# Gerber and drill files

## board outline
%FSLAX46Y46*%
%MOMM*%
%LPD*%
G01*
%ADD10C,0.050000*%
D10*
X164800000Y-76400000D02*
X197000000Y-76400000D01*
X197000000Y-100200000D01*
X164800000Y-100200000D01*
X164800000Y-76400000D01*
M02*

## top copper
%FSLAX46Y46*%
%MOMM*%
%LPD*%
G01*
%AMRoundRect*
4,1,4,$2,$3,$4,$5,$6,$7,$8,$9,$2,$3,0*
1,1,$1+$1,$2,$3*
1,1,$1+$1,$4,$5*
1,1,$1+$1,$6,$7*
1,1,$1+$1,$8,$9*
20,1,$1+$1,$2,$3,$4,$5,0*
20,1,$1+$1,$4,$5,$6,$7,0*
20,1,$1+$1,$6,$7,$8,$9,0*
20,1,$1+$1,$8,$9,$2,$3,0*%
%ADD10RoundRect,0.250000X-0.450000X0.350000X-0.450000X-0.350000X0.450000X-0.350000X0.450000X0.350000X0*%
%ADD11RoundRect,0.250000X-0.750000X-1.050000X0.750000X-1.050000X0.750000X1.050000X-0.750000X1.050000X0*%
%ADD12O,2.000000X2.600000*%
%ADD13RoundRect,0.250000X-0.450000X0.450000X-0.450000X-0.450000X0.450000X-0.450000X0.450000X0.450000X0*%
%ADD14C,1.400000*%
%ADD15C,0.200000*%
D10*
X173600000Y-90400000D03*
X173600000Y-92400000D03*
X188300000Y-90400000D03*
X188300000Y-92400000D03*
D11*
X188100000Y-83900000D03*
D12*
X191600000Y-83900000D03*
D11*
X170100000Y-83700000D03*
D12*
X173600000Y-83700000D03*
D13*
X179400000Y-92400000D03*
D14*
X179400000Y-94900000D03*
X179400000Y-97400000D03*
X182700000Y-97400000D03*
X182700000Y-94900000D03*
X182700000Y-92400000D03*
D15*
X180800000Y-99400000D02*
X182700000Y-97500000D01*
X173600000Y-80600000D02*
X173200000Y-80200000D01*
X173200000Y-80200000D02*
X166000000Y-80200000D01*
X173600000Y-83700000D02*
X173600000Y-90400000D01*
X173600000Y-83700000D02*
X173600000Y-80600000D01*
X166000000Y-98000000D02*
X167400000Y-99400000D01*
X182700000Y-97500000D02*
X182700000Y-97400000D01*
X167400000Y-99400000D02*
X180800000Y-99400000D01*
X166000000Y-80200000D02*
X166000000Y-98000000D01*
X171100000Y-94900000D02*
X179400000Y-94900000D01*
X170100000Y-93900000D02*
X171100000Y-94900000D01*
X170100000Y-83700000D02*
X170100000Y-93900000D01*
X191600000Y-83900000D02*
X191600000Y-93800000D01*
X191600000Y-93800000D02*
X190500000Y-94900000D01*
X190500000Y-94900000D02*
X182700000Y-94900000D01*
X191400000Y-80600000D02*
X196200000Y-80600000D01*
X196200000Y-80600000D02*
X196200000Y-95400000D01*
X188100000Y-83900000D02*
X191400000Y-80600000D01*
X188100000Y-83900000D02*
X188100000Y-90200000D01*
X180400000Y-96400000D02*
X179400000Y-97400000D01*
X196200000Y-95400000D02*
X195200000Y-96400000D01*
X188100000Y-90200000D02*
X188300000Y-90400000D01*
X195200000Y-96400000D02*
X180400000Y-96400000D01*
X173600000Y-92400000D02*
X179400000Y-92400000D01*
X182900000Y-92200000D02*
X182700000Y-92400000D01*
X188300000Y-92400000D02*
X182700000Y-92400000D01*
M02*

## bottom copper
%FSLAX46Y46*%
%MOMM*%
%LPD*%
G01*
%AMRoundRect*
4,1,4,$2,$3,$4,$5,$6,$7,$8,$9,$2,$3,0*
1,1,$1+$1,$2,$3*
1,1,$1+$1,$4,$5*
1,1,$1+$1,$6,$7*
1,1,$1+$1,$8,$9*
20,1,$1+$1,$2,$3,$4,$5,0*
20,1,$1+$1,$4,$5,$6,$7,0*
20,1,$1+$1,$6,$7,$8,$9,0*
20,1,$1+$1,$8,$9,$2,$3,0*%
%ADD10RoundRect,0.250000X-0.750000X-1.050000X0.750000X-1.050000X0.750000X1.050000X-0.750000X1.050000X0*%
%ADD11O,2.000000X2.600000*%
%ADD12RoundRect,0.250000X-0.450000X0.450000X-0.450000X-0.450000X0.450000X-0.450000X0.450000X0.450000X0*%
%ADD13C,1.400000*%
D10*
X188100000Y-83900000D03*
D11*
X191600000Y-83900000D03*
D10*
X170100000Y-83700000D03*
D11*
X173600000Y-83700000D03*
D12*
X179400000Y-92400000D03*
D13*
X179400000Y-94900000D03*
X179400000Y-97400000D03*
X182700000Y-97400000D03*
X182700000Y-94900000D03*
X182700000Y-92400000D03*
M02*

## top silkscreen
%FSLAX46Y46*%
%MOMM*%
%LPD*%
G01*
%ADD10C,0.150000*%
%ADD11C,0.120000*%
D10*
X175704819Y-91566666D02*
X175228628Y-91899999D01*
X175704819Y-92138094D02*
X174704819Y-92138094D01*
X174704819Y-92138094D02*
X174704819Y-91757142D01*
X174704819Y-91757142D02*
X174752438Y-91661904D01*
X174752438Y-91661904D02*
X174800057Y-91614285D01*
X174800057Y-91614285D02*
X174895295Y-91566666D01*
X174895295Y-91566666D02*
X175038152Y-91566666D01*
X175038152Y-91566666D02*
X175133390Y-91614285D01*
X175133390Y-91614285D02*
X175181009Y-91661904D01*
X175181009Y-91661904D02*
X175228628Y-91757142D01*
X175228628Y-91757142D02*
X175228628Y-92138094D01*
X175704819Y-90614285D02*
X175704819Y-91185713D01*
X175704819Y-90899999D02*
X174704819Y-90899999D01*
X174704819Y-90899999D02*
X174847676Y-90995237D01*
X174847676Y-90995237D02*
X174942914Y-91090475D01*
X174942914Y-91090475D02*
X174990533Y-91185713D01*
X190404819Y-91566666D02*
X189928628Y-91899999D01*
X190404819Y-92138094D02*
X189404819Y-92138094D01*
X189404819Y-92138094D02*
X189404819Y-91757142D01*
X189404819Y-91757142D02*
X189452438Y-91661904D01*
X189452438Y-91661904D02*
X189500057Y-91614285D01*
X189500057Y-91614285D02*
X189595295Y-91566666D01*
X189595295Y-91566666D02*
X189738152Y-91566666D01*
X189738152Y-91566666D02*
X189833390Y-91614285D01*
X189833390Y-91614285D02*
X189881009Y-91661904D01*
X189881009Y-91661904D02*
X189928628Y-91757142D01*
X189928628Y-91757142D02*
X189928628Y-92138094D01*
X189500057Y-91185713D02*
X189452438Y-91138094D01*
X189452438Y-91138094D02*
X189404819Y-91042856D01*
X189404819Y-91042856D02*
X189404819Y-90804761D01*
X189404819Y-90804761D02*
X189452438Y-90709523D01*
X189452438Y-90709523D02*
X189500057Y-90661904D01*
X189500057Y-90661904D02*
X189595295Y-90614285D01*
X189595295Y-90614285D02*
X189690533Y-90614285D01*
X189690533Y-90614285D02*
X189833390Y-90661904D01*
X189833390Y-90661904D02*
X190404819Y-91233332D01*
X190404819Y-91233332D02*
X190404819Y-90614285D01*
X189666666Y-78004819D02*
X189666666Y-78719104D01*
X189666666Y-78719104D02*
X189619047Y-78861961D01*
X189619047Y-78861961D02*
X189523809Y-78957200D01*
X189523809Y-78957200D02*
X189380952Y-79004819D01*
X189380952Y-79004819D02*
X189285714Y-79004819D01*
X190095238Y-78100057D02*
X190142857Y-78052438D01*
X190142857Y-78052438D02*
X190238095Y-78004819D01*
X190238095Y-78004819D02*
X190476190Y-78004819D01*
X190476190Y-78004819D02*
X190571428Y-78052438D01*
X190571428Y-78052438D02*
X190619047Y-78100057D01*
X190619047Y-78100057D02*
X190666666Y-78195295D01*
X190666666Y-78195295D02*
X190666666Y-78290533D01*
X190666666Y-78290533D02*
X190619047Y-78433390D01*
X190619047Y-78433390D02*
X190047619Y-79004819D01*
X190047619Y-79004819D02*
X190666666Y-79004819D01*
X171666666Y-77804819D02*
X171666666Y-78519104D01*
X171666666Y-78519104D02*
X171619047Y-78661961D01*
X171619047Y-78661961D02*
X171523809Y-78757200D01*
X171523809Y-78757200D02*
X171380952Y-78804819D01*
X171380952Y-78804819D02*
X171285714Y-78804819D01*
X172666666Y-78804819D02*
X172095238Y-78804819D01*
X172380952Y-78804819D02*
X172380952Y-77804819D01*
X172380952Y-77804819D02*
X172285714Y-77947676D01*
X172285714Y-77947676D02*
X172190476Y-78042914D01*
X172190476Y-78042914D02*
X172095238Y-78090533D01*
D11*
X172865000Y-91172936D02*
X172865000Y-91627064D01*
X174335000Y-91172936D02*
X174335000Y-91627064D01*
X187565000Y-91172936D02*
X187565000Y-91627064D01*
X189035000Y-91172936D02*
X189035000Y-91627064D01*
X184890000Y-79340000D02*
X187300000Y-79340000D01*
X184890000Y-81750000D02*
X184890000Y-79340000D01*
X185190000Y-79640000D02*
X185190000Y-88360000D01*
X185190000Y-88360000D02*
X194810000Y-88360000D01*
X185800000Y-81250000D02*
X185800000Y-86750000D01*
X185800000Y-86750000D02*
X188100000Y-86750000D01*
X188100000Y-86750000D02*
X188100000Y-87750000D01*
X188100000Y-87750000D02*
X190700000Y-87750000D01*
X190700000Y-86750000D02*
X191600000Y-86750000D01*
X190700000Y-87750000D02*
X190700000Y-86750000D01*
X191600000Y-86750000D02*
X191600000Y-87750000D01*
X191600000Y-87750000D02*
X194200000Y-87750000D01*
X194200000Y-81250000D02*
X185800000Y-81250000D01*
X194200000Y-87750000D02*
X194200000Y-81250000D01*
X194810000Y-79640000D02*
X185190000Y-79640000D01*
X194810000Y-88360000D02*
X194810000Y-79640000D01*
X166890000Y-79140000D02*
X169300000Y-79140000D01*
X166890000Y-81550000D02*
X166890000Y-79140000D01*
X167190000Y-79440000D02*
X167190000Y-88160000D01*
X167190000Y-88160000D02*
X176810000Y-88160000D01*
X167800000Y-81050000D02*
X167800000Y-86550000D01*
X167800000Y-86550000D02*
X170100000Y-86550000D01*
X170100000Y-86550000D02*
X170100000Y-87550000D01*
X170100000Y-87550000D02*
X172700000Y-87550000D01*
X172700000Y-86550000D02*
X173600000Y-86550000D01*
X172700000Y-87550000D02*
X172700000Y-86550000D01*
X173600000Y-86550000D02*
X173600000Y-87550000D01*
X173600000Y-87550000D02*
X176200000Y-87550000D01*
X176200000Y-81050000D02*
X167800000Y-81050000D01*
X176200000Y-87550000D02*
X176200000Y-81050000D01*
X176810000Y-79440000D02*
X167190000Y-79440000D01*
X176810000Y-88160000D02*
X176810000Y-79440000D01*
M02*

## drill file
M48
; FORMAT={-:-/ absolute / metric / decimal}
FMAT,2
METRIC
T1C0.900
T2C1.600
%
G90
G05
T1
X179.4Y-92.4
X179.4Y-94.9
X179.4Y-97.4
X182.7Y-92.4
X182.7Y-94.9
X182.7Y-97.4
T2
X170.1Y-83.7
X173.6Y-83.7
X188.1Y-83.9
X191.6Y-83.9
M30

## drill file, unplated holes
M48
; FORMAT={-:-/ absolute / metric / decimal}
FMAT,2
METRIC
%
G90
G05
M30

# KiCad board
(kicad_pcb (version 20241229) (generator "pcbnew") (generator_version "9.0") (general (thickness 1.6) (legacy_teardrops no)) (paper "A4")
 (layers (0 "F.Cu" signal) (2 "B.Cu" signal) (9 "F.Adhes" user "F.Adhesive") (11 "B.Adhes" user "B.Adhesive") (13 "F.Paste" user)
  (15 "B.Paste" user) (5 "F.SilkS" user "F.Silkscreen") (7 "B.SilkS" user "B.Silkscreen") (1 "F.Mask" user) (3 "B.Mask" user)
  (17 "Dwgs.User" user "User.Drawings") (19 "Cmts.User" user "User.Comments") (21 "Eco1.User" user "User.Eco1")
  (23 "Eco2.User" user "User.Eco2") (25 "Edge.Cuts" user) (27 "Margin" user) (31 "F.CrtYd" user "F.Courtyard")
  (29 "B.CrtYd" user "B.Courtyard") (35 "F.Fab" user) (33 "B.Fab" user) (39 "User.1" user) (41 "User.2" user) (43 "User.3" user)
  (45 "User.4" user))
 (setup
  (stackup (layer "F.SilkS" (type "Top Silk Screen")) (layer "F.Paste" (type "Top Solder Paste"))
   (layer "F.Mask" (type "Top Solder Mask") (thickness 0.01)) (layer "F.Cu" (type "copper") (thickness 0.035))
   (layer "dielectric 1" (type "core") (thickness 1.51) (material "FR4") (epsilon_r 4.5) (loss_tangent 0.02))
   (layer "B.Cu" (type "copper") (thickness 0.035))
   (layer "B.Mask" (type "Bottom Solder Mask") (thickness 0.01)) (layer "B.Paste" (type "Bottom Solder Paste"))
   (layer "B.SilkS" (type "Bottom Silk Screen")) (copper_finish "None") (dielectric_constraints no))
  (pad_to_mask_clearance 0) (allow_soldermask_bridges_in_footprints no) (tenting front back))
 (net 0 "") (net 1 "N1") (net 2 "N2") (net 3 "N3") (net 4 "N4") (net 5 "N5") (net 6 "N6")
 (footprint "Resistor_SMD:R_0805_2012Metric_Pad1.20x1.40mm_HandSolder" (layer "F.Cu") (at 173.6 91.4 -90)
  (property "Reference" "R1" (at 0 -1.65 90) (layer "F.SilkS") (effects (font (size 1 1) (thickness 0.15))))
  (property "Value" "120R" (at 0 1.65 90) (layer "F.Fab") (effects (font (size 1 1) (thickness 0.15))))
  (fp_line (start -0.227064 0.735) (end 0.227064 0.735) (stroke (width 0.12) (type solid)) (layer "F.SilkS"))
  (fp_line (start -0.227064 -0.735) (end 0.227064 -0.735) (stroke (width 0.12) (type solid)) (layer "F.SilkS"))
  (pad "1" smd roundrect (at -1 0 270) (size 1.2 1.4) (layers "F.Cu" "F.Mask" "F.Paste") (roundrect_rratio 0.208333) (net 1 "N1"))
  (pad "2" smd roundrect (at 1 0 270) (size 1.2 1.4) (layers "F.Cu" "F.Mask" "F.Paste") (roundrect_rratio 0.208333) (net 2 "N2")))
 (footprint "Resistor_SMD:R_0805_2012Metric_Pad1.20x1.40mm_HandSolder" (layer "F.Cu") (at 188.3 91.4 -90)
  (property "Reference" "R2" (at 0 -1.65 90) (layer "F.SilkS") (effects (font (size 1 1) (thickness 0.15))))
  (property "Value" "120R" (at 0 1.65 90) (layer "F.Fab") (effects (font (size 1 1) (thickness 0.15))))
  (fp_line (start -0.227064 0.735) (end 0.227064 0.735) (stroke (width 0.12) (type solid)) (layer "F.SilkS"))
  (fp_line (start -0.227064 -0.735) (end 0.227064 -0.735) (stroke (width 0.12) (type solid)) (layer "F.SilkS"))
  (pad "1" smd roundrect (at -1 0 270) (size 1.2 1.4) (layers "F.Cu" "F.Mask" "F.Paste") (roundrect_rratio 0.208333) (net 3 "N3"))
  (pad "2" smd roundrect (at 1 0 270) (size 1.2 1.4) (layers "F.Cu" "F.Mask" "F.Paste") (roundrect_rratio 0.208333) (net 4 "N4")))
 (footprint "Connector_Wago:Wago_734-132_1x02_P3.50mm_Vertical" (layer "F.Cu") (at 188.1 83.9)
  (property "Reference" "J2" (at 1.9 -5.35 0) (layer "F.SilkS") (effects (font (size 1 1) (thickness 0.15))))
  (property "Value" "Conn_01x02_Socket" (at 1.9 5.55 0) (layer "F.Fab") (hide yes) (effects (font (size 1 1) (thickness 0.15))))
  (fp_line (start -3.21 -4.56) (end -0.8 -4.56) (stroke (width 0.12) (type solid)) (layer "F.SilkS"))
  (fp_line (start -3.21 -2.15) (end -3.21 -4.56) (stroke (width 0.12) (type solid)) (layer "F.SilkS"))
  (fp_line (start -2.91 -4.26) (end -2.91 4.46) (stroke (width 0.12) (type solid)) (layer "F.SilkS"))
  (fp_line (start -2.91 4.46) (end 6.71 4.46) (stroke (width 0.12) (type solid)) (layer "F.SilkS"))
  (fp_line (start -2.3 -2.65) (end -2.3 2.85) (stroke (width 0.12) (type solid)) (layer "F.SilkS"))
  (fp_line (start -2.3 2.85) (end 0 2.85) (stroke (width 0.12) (type solid)) (layer "F.SilkS"))
  (fp_line (start 0 2.85) (end 0 3.85) (stroke (width 0.12) (type solid)) (layer "F.SilkS"))
  (fp_line (start 0 3.85) (end 2.6 3.85) (stroke (width 0.12) (type solid)) (layer "F.SilkS"))
  (fp_line (start 2.6 2.85) (end 3.5 2.85) (stroke (width 0.12) (type solid)) (layer "F.SilkS"))
  (fp_line (start 2.6 3.85) (end 2.6 2.85) (stroke (width 0.12) (type solid)) (layer "F.SilkS"))
  (fp_line (start 3.5 2.85) (end 3.5 3.85) (stroke (width 0.12) (type solid)) (layer "F.SilkS"))
  (fp_line (start 3.5 3.85) (end 6.1 3.85) (stroke (width 0.12) (type solid)) (layer "F.SilkS"))
  (fp_line (start 6.1 -2.65) (end -2.3 -2.65) (stroke (width 0.12) (type solid)) (layer "F.SilkS"))
  (fp_line (start 6.1 3.85) (end 6.1 -2.65) (stroke (width 0.12) (type solid)) (layer "F.SilkS"))
  (fp_line (start 6.71 -4.26) (end -2.91 -4.26) (stroke (width 0.12) (type solid)) (layer "F.SilkS"))
  (fp_line (start 6.71 4.46) (end 6.71 -4.26) (stroke (width 0.12) (type solid)) (layer "F.SilkS"))
  (pad "1" thru_hole roundrect (at 0 0) (size 2 2.6) (drill 1.6) (layers "*.Cu" "*.Mask") (remove_unused_layers no) (roundrect_rratio 0.125)
   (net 3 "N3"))
  (pad "2" thru_hole oval (at 3.5 0) (size 2 2.6) (drill 1.6) (layers "*.Cu" "*.Mask") (remove_unused_layers no) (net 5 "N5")))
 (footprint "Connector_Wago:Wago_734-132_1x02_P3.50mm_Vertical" (layer "F.Cu") (at 170.1 83.7)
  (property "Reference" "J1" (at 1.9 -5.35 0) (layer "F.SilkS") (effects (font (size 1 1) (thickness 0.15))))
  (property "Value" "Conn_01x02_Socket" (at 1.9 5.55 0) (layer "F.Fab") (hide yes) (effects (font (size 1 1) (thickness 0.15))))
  (fp_line (start -3.21 -4.56) (end -0.8 -4.56) (stroke (width 0.12) (type solid)) (layer "F.SilkS"))
  (fp_line (start -3.21 -2.15) (end -3.21 -4.56) (stroke (width 0.12) (type solid)) (layer "F.SilkS"))
  (fp_line (start -2.91 -4.26) (end -2.91 4.46) (stroke (width 0.12) (type solid)) (layer "F.SilkS"))
  (fp_line (start -2.91 4.46) (end 6.71 4.46) (stroke (width 0.12) (type solid)) (layer "F.SilkS"))
  (fp_line (start -2.3 -2.65) (end -2.3 2.85) (stroke (width 0.12) (type solid)) (layer "F.SilkS"))
  (fp_line (start -2.3 2.85) (end 0 2.85) (stroke (width 0.12) (type solid)) (layer "F.SilkS"))
  (fp_line (start 0 2.85) (end 0 3.85) (stroke (width 0.12) (type solid)) (layer "F.SilkS"))
  (fp_line (start 0 3.85) (end 2.6 3.85) (stroke (width 0.12) (type solid)) (layer "F.SilkS"))
  (fp_line (start 2.6 2.85) (end 3.5 2.85) (stroke (width 0.12) (type solid)) (layer "F.SilkS"))
  (fp_line (start 2.6 3.85) (end 2.6 2.85) (stroke (width 0.12) (type solid)) (layer "F.SilkS"))
  (fp_line (start 3.5 2.85) (end 3.5 3.85) (stroke (width 0.12) (type solid)) (layer "F.SilkS"))
  (fp_line (start 3.5 3.85) (end 6.1 3.85) (stroke (width 0.12) (type solid)) (layer "F.SilkS"))
  (fp_line (start 6.1 -2.65) (end -2.3 -2.65) (stroke (width 0.12) (type solid)) (layer "F.SilkS"))
  (fp_line (start 6.1 3.85) (end 6.1 -2.65) (stroke (width 0.12) (type solid)) (layer "F.SilkS"))
  (fp_line (start 6.71 -4.26) (end -2.91 -4.26) (stroke (width 0.12) (type solid)) (layer "F.SilkS"))
  (fp_line (start 6.71 4.46) (end 6.71 -4.26) (stroke (width 0.12) (type solid)) (layer "F.SilkS"))
  (pad "1" thru_hole roundrect (at 0 0) (size 2 2.6) (drill 1.6) (layers "*.Cu" "*.Mask") (remove_unused_layers no) (roundrect_rratio 0.125)
   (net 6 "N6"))
  (pad "2" thru_hole oval (at 3.5 0) (size 2 2.6) (drill 1.6) (layers "*.Cu" "*.Mask") (remove_unused_layers no) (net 1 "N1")))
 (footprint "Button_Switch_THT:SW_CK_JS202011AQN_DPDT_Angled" (layer "B.Cu") (at 179.4 92.4 -90)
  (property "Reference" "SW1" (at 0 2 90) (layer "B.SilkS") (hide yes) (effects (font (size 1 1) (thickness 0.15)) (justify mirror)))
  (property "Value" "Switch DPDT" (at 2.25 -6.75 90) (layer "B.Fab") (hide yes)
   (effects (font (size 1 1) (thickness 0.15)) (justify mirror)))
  (pad "1" thru_hole roundrect (at 0 0 270) (size 1.4 1.4) (drill 0.9) (layers "*.Cu" "*.Mask") (remove_unused_layers no)
   (roundrect_rratio 0.1785714286) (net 2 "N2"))
  (pad "2" thru_hole circle (at 2.5 0 270) (size 1.4 1.4) (drill 0.9) (layers "*.Cu" "*.Mask") (remove_unused_layers no) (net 6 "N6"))
  (pad "3" thru_hole circle (at 5 0 270) (size 1.4 1.4) (drill 0.9) (layers "*.Cu" "*.Mask") (remove_unused_layers no) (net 3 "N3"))
  (pad "4" thru_hole circle (at 5 -3.3 270) (size 1.4 1.4) (drill 0.9) (layers "*.Cu" "*.Mask") (remove_unused_layers no) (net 1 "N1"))
  (pad "5" thru_hole circle (at 2.5 -3.3 270) (size 1.4 1.4) (drill 0.9) (layers "*.Cu" "*.Mask") (remove_unused_layers no) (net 5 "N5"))
  (pad "6" thru_hole circle (at 0 -3.3 270) (size 1.4 1.4) (drill 0.9) (layers "*.Cu" "*.Mask") (remove_unused_layers no) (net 4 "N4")))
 (gr_rect (start 164.8 76.4) (end 197 100.2) (stroke (width 0.05) (type default)) (fill no) (layer "Edge.Cuts"))
 (segment (start 180.8 99.4) (end 182.7 97.5) (width 0.2) (layer "F.Cu") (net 1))
 (segment (start 173.6 80.6) (end 173.2 80.2) (width 0.2) (layer "F.Cu") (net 1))
 (segment (start 173.2 80.2) (end 166 80.2) (width 0.2) (layer "F.Cu") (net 1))
 (segment (start 173.6 83.7) (end 173.6 90.4) (width 0.2) (layer "F.Cu") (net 1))
 (segment (start 173.6 83.7) (end 173.6 80.6) (width 0.2) (layer "F.Cu") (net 1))
 (segment (start 166 98) (end 167.4 99.4) (width 0.2) (layer "F.Cu") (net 1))
 (segment (start 182.7 97.5) (end 182.7 97.4) (width 0.2) (layer "F.Cu") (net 1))
 (segment (start 167.4 99.4) (end 180.8 99.4) (width 0.2) (layer "F.Cu") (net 1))
 (segment (start 166 80.2) (end 166 98) (width 0.2) (layer "F.Cu") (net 1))
 (segment (start 171.1 94.9) (end 179.4 94.9) (width 0.2) (layer "F.Cu") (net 6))
 (segment (start 170.1 93.9) (end 171.1 94.9) (width 0.2) (layer "F.Cu") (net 6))
 (segment (start 170.1 83.7) (end 170.1 93.9) (width 0.2) (layer "F.Cu") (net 6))
 (segment (start 191.6 83.9) (end 191.6 93.8) (width 0.2) (layer "F.Cu") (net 5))
 (segment (start 191.6 93.8) (end 190.5 94.9) (width 0.2) (layer "F.Cu") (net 5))
 (segment (start 190.5 94.9) (end 182.7 94.9) (width 0.2) (layer "F.Cu") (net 5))
 (segment (start 191.4 80.6) (end 196.2 80.6) (width 0.2) (layer "F.Cu") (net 3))
 (segment (start 196.2 80.6) (end 196.2 95.4) (width 0.2) (layer "F.Cu") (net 3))
 (segment (start 188.1 83.9) (end 191.4 80.6) (width 0.2) (layer "F.Cu") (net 3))
 (segment (start 188.1 83.9) (end 188.1 90.2) (width 0.2) (layer "F.Cu") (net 3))
 (segment (start 180.4 96.4) (end 179.4 97.4) (width 0.2) (layer "F.Cu") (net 3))
 (segment (start 196.2 95.4) (end 195.2 96.4) (width 0.2) (layer "F.Cu") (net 3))
 (segment (start 188.1 90.2) (end 188.3 90.4) (width 0.2) (layer "F.Cu") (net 3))
 (segment (start 195.2 96.4) (end 180.4 96.4) (width 0.2) (layer "F.Cu") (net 3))
 (segment (start 173.6 92.4) (end 179.4 92.4) (width 0.2) (layer "F.Cu") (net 2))
 (segment (start 182.9 92.2) (end 182.7 92.4) (width 0.2) (layer "F.Cu") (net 4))
 (segment (start 188.3 92.4) (end 182.7 92.4) (width 0.2) (layer "F.Cu") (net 4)))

